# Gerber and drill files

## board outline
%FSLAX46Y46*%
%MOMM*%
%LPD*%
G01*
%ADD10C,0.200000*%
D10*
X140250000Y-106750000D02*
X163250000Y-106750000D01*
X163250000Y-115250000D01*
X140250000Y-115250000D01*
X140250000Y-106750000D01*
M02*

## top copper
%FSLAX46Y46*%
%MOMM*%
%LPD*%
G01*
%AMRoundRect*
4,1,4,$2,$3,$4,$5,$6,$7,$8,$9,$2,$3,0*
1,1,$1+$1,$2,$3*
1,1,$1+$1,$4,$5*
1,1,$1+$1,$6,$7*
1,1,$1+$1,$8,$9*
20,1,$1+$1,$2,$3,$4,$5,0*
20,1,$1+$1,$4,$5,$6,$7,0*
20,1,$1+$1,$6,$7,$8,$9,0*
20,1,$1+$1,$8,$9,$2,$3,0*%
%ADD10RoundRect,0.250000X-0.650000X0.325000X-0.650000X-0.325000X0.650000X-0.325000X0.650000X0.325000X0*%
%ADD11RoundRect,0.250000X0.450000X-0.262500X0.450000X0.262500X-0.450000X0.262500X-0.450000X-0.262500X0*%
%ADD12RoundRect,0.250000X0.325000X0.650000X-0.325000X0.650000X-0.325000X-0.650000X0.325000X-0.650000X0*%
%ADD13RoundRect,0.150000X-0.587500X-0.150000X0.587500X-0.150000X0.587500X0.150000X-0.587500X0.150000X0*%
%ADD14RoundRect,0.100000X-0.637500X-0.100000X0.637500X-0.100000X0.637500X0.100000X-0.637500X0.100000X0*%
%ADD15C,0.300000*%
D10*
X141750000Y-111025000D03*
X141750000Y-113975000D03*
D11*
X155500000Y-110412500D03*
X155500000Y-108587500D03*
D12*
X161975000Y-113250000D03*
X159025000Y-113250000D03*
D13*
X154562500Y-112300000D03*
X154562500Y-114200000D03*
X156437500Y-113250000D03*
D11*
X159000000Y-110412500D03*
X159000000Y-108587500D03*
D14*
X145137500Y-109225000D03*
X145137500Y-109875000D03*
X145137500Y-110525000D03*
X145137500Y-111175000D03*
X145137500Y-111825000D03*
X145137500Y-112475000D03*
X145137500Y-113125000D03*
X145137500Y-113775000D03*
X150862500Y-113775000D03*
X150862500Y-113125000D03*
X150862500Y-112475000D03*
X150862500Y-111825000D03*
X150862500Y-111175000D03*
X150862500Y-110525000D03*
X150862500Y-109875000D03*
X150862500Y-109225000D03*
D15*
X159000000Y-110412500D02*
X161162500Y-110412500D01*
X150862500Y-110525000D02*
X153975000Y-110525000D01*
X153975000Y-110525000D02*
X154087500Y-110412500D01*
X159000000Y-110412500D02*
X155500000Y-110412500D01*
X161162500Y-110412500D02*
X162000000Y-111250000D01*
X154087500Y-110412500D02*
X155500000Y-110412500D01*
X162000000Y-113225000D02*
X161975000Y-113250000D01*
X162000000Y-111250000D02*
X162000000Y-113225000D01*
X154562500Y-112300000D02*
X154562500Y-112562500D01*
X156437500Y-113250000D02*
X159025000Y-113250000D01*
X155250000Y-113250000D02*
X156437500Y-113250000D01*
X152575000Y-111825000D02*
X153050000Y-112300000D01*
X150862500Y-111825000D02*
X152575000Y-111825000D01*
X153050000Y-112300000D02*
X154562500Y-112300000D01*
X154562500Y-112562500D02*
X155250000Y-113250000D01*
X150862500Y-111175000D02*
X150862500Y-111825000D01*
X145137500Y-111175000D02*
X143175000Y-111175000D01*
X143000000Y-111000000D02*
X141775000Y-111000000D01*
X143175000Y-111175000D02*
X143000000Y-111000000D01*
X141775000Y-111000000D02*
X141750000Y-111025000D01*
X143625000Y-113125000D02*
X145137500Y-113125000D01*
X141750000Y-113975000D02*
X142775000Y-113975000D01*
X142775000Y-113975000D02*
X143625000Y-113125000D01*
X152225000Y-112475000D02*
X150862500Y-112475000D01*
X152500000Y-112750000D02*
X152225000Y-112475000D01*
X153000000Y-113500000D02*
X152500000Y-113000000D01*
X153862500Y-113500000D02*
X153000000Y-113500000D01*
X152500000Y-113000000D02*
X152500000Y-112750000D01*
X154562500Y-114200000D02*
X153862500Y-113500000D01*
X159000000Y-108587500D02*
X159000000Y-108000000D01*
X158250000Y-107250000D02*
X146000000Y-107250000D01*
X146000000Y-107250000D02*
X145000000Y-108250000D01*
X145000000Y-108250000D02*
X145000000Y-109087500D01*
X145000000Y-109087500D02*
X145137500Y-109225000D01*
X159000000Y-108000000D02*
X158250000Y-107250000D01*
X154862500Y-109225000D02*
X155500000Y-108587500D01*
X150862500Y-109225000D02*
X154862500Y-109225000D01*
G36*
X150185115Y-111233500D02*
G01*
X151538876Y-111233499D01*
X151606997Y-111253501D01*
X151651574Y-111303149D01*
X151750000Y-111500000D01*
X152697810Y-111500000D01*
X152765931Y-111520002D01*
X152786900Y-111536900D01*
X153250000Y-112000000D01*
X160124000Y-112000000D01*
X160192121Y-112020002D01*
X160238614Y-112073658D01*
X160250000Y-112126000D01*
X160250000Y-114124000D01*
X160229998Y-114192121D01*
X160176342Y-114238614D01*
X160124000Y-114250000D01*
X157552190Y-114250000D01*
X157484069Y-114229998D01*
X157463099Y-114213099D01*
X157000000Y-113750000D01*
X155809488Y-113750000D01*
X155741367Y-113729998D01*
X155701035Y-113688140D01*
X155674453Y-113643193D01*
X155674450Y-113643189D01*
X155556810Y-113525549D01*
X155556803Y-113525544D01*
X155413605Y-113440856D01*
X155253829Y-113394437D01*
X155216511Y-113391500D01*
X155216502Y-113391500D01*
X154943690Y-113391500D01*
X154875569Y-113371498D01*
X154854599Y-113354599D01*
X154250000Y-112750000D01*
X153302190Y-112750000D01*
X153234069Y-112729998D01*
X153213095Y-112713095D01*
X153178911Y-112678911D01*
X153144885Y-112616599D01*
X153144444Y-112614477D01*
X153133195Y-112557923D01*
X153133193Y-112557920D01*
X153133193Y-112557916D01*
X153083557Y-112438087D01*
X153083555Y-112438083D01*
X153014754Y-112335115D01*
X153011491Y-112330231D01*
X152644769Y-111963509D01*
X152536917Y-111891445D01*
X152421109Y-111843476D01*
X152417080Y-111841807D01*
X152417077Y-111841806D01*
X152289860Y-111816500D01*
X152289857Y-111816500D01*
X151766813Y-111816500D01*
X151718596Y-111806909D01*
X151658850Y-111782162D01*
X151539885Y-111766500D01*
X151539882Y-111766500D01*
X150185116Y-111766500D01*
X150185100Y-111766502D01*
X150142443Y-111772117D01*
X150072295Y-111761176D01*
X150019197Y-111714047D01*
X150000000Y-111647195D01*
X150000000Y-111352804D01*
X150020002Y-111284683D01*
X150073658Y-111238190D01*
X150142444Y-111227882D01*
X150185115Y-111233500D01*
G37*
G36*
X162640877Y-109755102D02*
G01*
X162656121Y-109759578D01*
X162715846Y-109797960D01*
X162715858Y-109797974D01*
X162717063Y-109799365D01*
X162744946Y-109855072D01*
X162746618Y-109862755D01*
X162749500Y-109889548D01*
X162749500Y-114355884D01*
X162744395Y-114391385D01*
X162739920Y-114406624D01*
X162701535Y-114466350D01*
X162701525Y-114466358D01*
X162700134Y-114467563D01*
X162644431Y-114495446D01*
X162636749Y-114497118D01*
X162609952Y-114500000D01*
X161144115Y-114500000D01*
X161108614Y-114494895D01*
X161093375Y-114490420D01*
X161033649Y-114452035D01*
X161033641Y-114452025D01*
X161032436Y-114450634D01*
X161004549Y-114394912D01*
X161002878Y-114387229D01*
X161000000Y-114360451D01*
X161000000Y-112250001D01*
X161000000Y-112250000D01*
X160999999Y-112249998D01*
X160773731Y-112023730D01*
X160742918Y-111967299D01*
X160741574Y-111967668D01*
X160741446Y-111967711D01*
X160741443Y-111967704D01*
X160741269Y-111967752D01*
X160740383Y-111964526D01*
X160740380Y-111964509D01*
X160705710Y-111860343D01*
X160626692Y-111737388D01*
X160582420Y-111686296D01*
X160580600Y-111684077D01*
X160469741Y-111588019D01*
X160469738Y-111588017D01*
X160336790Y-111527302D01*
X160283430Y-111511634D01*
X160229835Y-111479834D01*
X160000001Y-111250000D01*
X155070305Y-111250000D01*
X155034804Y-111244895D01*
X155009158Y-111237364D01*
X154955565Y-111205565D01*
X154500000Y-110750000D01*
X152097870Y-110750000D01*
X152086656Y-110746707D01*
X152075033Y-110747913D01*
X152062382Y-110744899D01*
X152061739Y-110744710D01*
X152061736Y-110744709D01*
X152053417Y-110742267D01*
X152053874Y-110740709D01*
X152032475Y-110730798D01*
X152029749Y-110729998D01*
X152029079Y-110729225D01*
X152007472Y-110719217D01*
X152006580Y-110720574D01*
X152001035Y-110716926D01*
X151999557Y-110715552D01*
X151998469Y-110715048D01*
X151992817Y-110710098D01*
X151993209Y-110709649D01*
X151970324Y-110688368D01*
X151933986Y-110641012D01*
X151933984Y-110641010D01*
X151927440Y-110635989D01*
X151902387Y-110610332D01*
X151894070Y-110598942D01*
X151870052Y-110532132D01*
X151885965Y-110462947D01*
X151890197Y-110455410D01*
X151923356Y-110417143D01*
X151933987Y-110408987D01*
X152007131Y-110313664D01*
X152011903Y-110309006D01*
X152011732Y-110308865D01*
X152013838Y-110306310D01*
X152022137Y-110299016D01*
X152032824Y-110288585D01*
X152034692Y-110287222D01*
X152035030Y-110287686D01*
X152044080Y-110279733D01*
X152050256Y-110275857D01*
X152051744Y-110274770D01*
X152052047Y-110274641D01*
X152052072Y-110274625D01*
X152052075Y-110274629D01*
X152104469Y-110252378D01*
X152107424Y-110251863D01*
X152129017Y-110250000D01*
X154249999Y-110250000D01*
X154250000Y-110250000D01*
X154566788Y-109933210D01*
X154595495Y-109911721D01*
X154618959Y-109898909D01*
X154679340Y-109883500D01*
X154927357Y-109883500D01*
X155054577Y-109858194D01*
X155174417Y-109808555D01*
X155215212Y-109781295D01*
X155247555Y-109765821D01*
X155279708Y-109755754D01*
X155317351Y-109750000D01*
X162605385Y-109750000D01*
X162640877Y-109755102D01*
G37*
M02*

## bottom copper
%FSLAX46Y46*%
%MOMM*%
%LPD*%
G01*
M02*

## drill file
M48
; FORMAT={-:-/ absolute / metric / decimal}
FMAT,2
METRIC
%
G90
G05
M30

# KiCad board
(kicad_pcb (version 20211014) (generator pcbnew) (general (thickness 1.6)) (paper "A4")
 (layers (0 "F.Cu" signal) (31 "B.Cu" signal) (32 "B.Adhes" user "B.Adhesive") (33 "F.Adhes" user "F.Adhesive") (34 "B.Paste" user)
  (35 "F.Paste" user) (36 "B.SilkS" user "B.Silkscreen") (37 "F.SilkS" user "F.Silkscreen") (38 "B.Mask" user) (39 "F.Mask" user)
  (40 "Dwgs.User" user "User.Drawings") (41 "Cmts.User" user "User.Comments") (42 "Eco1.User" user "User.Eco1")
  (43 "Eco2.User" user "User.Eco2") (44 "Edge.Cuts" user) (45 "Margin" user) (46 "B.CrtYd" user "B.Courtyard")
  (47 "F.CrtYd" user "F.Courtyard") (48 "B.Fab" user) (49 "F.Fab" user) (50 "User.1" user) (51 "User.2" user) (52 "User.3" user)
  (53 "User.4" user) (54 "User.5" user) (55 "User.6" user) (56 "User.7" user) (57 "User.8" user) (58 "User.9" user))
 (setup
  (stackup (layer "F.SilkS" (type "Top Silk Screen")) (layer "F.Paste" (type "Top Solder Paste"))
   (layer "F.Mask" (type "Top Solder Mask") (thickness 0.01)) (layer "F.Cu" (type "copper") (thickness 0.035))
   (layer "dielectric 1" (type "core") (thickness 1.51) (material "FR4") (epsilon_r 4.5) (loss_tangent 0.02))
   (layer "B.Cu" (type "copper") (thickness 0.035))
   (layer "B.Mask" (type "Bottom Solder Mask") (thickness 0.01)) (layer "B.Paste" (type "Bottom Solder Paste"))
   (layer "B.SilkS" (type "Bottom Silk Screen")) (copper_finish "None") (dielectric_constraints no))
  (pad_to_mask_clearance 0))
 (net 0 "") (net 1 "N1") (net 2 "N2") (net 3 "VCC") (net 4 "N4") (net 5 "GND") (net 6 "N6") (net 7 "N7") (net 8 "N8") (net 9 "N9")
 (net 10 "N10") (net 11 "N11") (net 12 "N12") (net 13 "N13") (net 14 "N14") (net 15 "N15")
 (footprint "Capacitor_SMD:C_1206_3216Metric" (layer "F.Cu") (at 141.75 112.5 -90)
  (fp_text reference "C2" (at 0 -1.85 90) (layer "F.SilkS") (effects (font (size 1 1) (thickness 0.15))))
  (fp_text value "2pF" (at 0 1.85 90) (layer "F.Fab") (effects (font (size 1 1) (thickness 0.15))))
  (pad "1" smd roundrect (at -1.475 0 270) (size 1.15 1.8) (layers "F.Cu" "F.Paste" "F.Mask") (roundrect_rratio 0.217391) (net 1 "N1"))
  (pad "2" smd roundrect (at 1.475 0 270) (size 1.15 1.8) (layers "F.Cu" "F.Paste" "F.Mask") (roundrect_rratio 0.217391) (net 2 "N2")))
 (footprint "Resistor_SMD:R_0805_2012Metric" (layer "F.Cu") (at 155.5 109.5 90)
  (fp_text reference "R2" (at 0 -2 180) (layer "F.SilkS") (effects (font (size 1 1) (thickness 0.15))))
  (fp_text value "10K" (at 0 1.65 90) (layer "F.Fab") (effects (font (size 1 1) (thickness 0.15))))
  (pad "1" smd roundrect (at -0.9125 0 90) (size 1.025 1.4) (layers "F.Cu" "F.Paste" "F.Mask") (roundrect_rratio 0.243902) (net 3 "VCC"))
  (pad "2" smd roundrect (at 0.9125 0 90) (size 1.025 1.4) (layers "F.Cu" "F.Paste" "F.Mask") (roundrect_rratio 0.243902) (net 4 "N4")))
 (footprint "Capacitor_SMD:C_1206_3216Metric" (layer "F.Cu") (at 160.5 113.25 180)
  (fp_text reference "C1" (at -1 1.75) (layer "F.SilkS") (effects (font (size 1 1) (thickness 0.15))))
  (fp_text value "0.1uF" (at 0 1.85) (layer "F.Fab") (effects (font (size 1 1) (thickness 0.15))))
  (pad "1" smd roundrect (at -1.475 0 180) (size 1.15 1.8) (layers "F.Cu" "F.Paste" "F.Mask") (roundrect_rratio 0.217391) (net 3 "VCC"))
  (pad "2" smd roundrect (at 1.475 0 180) (size 1.15 1.8) (layers "F.Cu" "F.Paste" "F.Mask") (roundrect_rratio 0.217391) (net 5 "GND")))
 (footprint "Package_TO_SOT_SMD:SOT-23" (layer "F.Cu") (at 155.5 113.25)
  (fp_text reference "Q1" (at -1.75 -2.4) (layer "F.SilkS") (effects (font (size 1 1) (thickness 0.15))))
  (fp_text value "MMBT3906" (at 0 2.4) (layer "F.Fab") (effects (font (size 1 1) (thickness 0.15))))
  (pad "1" smd roundrect (at -0.9375 -0.95) (size 1.475 0.6) (layers "F.Cu" "F.Paste" "F.Mask") (roundrect_rratio 0.25) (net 5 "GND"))
  (pad "2" smd roundrect (at -0.9375 0.95) (size 1.475 0.6) (layers "F.Cu" "F.Paste" "F.Mask") (roundrect_rratio 0.25) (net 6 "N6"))
  (pad "3" smd roundrect (at 0.9375 0) (size 1.475 0.6) (layers "F.Cu" "F.Paste" "F.Mask") (roundrect_rratio 0.25) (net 5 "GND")))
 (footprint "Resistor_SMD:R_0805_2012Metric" (layer "F.Cu") (at 159 109.5 90)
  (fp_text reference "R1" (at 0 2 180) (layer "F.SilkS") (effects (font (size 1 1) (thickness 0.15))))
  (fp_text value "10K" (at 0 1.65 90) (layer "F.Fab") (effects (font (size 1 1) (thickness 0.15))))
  (pad "1" smd roundrect (at -0.9125 0 90) (size 1.025 1.4) (layers "F.Cu" "F.Paste" "F.Mask") (roundrect_rratio 0.243902) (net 3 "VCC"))
  (pad "2" smd roundrect (at 0.9125 0 90) (size 1.025 1.4) (layers "F.Cu" "F.Paste" "F.Mask") (roundrect_rratio 0.243902) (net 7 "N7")))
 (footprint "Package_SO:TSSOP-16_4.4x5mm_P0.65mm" (layer "F.Cu") (at 148 111.5)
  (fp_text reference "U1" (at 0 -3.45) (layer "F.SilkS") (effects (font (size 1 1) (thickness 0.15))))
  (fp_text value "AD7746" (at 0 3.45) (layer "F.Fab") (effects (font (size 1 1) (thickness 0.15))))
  (pad "1" smd roundrect (at -2.8625 -2.275) (size 1.475 0.4) (layers "F.Cu" "F.Paste" "F.Mask") (roundrect_rratio 0.25) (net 7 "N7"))
  (pad "2" smd roundrect (at -2.8625 -1.625) (size 1.475 0.4) (layers "F.Cu" "F.Paste" "F.Mask") (roundrect_rratio 0.25) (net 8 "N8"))
  (pad "3" smd roundrect (at -2.8625 -0.975) (size 1.475 0.4) (layers "F.Cu" "F.Paste" "F.Mask") (roundrect_rratio 0.25) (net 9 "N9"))
  (pad "4" smd roundrect (at -2.8625 -0.325) (size 1.475 0.4) (layers "F.Cu" "F.Paste" "F.Mask") (roundrect_rratio 0.25) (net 1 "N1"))
  (pad "5" smd roundrect (at -2.8625 0.325) (size 1.475 0.4) (layers "F.Cu" "F.Paste" "F.Mask") (roundrect_rratio 0.25) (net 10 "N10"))
  (pad "6" smd roundrect (at -2.8625 0.975) (size 1.475 0.4) (layers "F.Cu" "F.Paste" "F.Mask") (roundrect_rratio 0.25) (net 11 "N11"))
  (pad "7" smd roundrect (at -2.8625 1.625) (size 1.475 0.4) (layers "F.Cu" "F.Paste" "F.Mask") (roundrect_rratio 0.25) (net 2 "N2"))
  (pad "8" smd roundrect (at -2.8625 2.275) (size 1.475 0.4) (layers "F.Cu" "F.Paste" "F.Mask") (roundrect_rratio 0.25) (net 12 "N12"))
  (pad "9" smd roundrect (at 2.8625 2.275) (size 1.475 0.4) (layers "F.Cu" "F.Paste" "F.Mask") (roundrect_rratio 0.25) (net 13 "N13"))
  (pad "10" smd roundrect (at 2.8625 1.625) (size 1.475 0.4) (layers "F.Cu" "F.Paste" "F.Mask") (roundrect_rratio 0.25) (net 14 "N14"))
  (pad "11" smd roundrect (at 2.8625 0.975) (size 1.475 0.4) (layers "F.Cu" "F.Paste" "F.Mask") (roundrect_rratio 0.25) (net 6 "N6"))
  (pad "12" smd roundrect (at 2.8625 0.325) (size 1.475 0.4) (layers "F.Cu" "F.Paste" "F.Mask") (roundrect_rratio 0.25) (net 5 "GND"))
  (pad "13" smd roundrect (at 2.8625 -0.325) (size 1.475 0.4) (layers "F.Cu" "F.Paste" "F.Mask") (roundrect_rratio 0.25) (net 5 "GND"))
  (pad "14" smd roundrect (at 2.8625 -0.975) (size 1.475 0.4) (layers "F.Cu" "F.Paste" "F.Mask") (roundrect_rratio 0.25) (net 3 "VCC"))
  (pad "15" smd roundrect (at 2.8625 -1.625) (size 1.475 0.4) (layers "F.Cu" "F.Paste" "F.Mask") (roundrect_rratio 0.25) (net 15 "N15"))
  (pad "16" smd roundrect (at 2.8625 -2.275) (size 1.475 0.4) (layers "F.Cu" "F.Paste" "F.Mask") (roundrect_rratio 0.25) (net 4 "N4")))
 (gr_rect (start 140.25 115.25) (end 163.25 106.75) (layer "Edge.Cuts") (width 0.2) (fill none))
 (segment (start 159 110.4125) (end 161.1625 110.4125) (width 0.3) (layer "F.Cu") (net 3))
 (segment (start 150.8625 110.525) (end 153.975 110.525) (width 0.3) (layer "F.Cu") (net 3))
 (segment (start 153.975 110.525) (end 154.0875 110.4125) (width 0.3) (layer "F.Cu") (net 3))
 (segment (start 159 110.4125) (end 155.5 110.4125) (width 0.3) (layer "F.Cu") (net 3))
 (segment (start 161.1625 110.4125) (end 162 111.25) (width 0.3) (layer "F.Cu") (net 3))
 (segment (start 154.0875 110.4125) (end 155.5 110.4125) (width 0.3) (layer "F.Cu") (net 3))
 (segment (start 162 113.225) (end 161.975 113.25) (width 0.3) (layer "F.Cu") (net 3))
 (segment (start 162 111.25) (end 162 113.225) (width 0.3) (layer "F.Cu") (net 3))
 (segment (start 154.5625 112.3) (end 154.5625 112.5625) (width 0.3) (layer "F.Cu") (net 5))
 (segment (start 156.4375 113.25) (end 159.025 113.25) (width 0.3) (layer "F.Cu") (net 5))
 (segment (start 155.25 113.25) (end 156.4375 113.25) (width 0.3) (layer "F.Cu") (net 5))
 (segment (start 152.575 111.825) (end 153.05 112.3) (width 0.3) (layer "F.Cu") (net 5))
 (segment (start 150.8625 111.825) (end 152.575 111.825) (width 0.3) (layer "F.Cu") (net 5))
 (segment (start 153.05 112.3) (end 154.5625 112.3) (width 0.3) (layer "F.Cu") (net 5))
 (segment (start 154.5625 112.5625) (end 155.25 113.25) (width 0.3) (layer "F.Cu") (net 5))
 (segment (start 150.8625 111.175) (end 150.8625 111.825) (width 0.3) (layer "F.Cu") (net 5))
 (segment (start 145.1375 111.175) (end 143.175 111.175) (width 0.3) (layer "F.Cu") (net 1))
 (segment (start 143 111) (end 141.775 111) (width 0.3) (layer "F.Cu") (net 1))
 (segment (start 143.175 111.175) (end 143 111) (width 0.3) (layer "F.Cu") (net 1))
 (segment (start 141.775 111) (end 141.75 111.025) (width 0.3) (layer "F.Cu") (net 1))
 (segment (start 143.625 113.125) (end 145.1375 113.125) (width 0.3) (layer "F.Cu") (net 2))
 (segment (start 141.75 113.975) (end 142.775 113.975) (width 0.3) (layer "F.Cu") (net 2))
 (segment (start 142.775 113.975) (end 143.625 113.125) (width 0.3) (layer "F.Cu") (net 2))
 (segment (start 152.225 112.475) (end 150.8625 112.475) (width 0.3) (layer "F.Cu") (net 6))
 (segment (start 152.5 112.75) (end 152.225 112.475) (width 0.3) (layer "F.Cu") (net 6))
 (segment (start 153 113.5) (end 152.5 113) (width 0.3) (layer "F.Cu") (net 6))
 (segment (start 153.8625 113.5) (end 153 113.5) (width 0.3) (layer "F.Cu") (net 6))
 (segment (start 152.5 113) (end 152.5 112.75) (width 0.3) (layer "F.Cu") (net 6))
 (segment (start 154.5625 114.2) (end 153.8625 113.5) (width 0.3) (layer "F.Cu") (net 6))
 (segment (start 159 108.5875) (end 159 108) (width 0.3) (layer "F.Cu") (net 7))
 (segment (start 158.25 107.25) (end 146 107.25) (width 0.3) (layer "F.Cu") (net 7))
 (segment (start 146 107.25) (end 145 108.25) (width 0.3) (layer "F.Cu") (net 7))
 (segment (start 145 108.25) (end 145 109.0875) (width 0.3) (layer "F.Cu") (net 7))
 (segment (start 145 109.0875) (end 145.1375 109.225) (width 0.3) (layer "F.Cu") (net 7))
 (segment (start 159 108) (end 158.25 107.25) (width 0.3) (layer "F.Cu") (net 7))
 (segment (start 154.8625 109.225) (end 155.5 108.5875) (width 0.3) (layer "F.Cu") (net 4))
 (segment (start 150.8625 109.225) (end 154.8625 109.225) (width 0.3) (layer "F.Cu") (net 4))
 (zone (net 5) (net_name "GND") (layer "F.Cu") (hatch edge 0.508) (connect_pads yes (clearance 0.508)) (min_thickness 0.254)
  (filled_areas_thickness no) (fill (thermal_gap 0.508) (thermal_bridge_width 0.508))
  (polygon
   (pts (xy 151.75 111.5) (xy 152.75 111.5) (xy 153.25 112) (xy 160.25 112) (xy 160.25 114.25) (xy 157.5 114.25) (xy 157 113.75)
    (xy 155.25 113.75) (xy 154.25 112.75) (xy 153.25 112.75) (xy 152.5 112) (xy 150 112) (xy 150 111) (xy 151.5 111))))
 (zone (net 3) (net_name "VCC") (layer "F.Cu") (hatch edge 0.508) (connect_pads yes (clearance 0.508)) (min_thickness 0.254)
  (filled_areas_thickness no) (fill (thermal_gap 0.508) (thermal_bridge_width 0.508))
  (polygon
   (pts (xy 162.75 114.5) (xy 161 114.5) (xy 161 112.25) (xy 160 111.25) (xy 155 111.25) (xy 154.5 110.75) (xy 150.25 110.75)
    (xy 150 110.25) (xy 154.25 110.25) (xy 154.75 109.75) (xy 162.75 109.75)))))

